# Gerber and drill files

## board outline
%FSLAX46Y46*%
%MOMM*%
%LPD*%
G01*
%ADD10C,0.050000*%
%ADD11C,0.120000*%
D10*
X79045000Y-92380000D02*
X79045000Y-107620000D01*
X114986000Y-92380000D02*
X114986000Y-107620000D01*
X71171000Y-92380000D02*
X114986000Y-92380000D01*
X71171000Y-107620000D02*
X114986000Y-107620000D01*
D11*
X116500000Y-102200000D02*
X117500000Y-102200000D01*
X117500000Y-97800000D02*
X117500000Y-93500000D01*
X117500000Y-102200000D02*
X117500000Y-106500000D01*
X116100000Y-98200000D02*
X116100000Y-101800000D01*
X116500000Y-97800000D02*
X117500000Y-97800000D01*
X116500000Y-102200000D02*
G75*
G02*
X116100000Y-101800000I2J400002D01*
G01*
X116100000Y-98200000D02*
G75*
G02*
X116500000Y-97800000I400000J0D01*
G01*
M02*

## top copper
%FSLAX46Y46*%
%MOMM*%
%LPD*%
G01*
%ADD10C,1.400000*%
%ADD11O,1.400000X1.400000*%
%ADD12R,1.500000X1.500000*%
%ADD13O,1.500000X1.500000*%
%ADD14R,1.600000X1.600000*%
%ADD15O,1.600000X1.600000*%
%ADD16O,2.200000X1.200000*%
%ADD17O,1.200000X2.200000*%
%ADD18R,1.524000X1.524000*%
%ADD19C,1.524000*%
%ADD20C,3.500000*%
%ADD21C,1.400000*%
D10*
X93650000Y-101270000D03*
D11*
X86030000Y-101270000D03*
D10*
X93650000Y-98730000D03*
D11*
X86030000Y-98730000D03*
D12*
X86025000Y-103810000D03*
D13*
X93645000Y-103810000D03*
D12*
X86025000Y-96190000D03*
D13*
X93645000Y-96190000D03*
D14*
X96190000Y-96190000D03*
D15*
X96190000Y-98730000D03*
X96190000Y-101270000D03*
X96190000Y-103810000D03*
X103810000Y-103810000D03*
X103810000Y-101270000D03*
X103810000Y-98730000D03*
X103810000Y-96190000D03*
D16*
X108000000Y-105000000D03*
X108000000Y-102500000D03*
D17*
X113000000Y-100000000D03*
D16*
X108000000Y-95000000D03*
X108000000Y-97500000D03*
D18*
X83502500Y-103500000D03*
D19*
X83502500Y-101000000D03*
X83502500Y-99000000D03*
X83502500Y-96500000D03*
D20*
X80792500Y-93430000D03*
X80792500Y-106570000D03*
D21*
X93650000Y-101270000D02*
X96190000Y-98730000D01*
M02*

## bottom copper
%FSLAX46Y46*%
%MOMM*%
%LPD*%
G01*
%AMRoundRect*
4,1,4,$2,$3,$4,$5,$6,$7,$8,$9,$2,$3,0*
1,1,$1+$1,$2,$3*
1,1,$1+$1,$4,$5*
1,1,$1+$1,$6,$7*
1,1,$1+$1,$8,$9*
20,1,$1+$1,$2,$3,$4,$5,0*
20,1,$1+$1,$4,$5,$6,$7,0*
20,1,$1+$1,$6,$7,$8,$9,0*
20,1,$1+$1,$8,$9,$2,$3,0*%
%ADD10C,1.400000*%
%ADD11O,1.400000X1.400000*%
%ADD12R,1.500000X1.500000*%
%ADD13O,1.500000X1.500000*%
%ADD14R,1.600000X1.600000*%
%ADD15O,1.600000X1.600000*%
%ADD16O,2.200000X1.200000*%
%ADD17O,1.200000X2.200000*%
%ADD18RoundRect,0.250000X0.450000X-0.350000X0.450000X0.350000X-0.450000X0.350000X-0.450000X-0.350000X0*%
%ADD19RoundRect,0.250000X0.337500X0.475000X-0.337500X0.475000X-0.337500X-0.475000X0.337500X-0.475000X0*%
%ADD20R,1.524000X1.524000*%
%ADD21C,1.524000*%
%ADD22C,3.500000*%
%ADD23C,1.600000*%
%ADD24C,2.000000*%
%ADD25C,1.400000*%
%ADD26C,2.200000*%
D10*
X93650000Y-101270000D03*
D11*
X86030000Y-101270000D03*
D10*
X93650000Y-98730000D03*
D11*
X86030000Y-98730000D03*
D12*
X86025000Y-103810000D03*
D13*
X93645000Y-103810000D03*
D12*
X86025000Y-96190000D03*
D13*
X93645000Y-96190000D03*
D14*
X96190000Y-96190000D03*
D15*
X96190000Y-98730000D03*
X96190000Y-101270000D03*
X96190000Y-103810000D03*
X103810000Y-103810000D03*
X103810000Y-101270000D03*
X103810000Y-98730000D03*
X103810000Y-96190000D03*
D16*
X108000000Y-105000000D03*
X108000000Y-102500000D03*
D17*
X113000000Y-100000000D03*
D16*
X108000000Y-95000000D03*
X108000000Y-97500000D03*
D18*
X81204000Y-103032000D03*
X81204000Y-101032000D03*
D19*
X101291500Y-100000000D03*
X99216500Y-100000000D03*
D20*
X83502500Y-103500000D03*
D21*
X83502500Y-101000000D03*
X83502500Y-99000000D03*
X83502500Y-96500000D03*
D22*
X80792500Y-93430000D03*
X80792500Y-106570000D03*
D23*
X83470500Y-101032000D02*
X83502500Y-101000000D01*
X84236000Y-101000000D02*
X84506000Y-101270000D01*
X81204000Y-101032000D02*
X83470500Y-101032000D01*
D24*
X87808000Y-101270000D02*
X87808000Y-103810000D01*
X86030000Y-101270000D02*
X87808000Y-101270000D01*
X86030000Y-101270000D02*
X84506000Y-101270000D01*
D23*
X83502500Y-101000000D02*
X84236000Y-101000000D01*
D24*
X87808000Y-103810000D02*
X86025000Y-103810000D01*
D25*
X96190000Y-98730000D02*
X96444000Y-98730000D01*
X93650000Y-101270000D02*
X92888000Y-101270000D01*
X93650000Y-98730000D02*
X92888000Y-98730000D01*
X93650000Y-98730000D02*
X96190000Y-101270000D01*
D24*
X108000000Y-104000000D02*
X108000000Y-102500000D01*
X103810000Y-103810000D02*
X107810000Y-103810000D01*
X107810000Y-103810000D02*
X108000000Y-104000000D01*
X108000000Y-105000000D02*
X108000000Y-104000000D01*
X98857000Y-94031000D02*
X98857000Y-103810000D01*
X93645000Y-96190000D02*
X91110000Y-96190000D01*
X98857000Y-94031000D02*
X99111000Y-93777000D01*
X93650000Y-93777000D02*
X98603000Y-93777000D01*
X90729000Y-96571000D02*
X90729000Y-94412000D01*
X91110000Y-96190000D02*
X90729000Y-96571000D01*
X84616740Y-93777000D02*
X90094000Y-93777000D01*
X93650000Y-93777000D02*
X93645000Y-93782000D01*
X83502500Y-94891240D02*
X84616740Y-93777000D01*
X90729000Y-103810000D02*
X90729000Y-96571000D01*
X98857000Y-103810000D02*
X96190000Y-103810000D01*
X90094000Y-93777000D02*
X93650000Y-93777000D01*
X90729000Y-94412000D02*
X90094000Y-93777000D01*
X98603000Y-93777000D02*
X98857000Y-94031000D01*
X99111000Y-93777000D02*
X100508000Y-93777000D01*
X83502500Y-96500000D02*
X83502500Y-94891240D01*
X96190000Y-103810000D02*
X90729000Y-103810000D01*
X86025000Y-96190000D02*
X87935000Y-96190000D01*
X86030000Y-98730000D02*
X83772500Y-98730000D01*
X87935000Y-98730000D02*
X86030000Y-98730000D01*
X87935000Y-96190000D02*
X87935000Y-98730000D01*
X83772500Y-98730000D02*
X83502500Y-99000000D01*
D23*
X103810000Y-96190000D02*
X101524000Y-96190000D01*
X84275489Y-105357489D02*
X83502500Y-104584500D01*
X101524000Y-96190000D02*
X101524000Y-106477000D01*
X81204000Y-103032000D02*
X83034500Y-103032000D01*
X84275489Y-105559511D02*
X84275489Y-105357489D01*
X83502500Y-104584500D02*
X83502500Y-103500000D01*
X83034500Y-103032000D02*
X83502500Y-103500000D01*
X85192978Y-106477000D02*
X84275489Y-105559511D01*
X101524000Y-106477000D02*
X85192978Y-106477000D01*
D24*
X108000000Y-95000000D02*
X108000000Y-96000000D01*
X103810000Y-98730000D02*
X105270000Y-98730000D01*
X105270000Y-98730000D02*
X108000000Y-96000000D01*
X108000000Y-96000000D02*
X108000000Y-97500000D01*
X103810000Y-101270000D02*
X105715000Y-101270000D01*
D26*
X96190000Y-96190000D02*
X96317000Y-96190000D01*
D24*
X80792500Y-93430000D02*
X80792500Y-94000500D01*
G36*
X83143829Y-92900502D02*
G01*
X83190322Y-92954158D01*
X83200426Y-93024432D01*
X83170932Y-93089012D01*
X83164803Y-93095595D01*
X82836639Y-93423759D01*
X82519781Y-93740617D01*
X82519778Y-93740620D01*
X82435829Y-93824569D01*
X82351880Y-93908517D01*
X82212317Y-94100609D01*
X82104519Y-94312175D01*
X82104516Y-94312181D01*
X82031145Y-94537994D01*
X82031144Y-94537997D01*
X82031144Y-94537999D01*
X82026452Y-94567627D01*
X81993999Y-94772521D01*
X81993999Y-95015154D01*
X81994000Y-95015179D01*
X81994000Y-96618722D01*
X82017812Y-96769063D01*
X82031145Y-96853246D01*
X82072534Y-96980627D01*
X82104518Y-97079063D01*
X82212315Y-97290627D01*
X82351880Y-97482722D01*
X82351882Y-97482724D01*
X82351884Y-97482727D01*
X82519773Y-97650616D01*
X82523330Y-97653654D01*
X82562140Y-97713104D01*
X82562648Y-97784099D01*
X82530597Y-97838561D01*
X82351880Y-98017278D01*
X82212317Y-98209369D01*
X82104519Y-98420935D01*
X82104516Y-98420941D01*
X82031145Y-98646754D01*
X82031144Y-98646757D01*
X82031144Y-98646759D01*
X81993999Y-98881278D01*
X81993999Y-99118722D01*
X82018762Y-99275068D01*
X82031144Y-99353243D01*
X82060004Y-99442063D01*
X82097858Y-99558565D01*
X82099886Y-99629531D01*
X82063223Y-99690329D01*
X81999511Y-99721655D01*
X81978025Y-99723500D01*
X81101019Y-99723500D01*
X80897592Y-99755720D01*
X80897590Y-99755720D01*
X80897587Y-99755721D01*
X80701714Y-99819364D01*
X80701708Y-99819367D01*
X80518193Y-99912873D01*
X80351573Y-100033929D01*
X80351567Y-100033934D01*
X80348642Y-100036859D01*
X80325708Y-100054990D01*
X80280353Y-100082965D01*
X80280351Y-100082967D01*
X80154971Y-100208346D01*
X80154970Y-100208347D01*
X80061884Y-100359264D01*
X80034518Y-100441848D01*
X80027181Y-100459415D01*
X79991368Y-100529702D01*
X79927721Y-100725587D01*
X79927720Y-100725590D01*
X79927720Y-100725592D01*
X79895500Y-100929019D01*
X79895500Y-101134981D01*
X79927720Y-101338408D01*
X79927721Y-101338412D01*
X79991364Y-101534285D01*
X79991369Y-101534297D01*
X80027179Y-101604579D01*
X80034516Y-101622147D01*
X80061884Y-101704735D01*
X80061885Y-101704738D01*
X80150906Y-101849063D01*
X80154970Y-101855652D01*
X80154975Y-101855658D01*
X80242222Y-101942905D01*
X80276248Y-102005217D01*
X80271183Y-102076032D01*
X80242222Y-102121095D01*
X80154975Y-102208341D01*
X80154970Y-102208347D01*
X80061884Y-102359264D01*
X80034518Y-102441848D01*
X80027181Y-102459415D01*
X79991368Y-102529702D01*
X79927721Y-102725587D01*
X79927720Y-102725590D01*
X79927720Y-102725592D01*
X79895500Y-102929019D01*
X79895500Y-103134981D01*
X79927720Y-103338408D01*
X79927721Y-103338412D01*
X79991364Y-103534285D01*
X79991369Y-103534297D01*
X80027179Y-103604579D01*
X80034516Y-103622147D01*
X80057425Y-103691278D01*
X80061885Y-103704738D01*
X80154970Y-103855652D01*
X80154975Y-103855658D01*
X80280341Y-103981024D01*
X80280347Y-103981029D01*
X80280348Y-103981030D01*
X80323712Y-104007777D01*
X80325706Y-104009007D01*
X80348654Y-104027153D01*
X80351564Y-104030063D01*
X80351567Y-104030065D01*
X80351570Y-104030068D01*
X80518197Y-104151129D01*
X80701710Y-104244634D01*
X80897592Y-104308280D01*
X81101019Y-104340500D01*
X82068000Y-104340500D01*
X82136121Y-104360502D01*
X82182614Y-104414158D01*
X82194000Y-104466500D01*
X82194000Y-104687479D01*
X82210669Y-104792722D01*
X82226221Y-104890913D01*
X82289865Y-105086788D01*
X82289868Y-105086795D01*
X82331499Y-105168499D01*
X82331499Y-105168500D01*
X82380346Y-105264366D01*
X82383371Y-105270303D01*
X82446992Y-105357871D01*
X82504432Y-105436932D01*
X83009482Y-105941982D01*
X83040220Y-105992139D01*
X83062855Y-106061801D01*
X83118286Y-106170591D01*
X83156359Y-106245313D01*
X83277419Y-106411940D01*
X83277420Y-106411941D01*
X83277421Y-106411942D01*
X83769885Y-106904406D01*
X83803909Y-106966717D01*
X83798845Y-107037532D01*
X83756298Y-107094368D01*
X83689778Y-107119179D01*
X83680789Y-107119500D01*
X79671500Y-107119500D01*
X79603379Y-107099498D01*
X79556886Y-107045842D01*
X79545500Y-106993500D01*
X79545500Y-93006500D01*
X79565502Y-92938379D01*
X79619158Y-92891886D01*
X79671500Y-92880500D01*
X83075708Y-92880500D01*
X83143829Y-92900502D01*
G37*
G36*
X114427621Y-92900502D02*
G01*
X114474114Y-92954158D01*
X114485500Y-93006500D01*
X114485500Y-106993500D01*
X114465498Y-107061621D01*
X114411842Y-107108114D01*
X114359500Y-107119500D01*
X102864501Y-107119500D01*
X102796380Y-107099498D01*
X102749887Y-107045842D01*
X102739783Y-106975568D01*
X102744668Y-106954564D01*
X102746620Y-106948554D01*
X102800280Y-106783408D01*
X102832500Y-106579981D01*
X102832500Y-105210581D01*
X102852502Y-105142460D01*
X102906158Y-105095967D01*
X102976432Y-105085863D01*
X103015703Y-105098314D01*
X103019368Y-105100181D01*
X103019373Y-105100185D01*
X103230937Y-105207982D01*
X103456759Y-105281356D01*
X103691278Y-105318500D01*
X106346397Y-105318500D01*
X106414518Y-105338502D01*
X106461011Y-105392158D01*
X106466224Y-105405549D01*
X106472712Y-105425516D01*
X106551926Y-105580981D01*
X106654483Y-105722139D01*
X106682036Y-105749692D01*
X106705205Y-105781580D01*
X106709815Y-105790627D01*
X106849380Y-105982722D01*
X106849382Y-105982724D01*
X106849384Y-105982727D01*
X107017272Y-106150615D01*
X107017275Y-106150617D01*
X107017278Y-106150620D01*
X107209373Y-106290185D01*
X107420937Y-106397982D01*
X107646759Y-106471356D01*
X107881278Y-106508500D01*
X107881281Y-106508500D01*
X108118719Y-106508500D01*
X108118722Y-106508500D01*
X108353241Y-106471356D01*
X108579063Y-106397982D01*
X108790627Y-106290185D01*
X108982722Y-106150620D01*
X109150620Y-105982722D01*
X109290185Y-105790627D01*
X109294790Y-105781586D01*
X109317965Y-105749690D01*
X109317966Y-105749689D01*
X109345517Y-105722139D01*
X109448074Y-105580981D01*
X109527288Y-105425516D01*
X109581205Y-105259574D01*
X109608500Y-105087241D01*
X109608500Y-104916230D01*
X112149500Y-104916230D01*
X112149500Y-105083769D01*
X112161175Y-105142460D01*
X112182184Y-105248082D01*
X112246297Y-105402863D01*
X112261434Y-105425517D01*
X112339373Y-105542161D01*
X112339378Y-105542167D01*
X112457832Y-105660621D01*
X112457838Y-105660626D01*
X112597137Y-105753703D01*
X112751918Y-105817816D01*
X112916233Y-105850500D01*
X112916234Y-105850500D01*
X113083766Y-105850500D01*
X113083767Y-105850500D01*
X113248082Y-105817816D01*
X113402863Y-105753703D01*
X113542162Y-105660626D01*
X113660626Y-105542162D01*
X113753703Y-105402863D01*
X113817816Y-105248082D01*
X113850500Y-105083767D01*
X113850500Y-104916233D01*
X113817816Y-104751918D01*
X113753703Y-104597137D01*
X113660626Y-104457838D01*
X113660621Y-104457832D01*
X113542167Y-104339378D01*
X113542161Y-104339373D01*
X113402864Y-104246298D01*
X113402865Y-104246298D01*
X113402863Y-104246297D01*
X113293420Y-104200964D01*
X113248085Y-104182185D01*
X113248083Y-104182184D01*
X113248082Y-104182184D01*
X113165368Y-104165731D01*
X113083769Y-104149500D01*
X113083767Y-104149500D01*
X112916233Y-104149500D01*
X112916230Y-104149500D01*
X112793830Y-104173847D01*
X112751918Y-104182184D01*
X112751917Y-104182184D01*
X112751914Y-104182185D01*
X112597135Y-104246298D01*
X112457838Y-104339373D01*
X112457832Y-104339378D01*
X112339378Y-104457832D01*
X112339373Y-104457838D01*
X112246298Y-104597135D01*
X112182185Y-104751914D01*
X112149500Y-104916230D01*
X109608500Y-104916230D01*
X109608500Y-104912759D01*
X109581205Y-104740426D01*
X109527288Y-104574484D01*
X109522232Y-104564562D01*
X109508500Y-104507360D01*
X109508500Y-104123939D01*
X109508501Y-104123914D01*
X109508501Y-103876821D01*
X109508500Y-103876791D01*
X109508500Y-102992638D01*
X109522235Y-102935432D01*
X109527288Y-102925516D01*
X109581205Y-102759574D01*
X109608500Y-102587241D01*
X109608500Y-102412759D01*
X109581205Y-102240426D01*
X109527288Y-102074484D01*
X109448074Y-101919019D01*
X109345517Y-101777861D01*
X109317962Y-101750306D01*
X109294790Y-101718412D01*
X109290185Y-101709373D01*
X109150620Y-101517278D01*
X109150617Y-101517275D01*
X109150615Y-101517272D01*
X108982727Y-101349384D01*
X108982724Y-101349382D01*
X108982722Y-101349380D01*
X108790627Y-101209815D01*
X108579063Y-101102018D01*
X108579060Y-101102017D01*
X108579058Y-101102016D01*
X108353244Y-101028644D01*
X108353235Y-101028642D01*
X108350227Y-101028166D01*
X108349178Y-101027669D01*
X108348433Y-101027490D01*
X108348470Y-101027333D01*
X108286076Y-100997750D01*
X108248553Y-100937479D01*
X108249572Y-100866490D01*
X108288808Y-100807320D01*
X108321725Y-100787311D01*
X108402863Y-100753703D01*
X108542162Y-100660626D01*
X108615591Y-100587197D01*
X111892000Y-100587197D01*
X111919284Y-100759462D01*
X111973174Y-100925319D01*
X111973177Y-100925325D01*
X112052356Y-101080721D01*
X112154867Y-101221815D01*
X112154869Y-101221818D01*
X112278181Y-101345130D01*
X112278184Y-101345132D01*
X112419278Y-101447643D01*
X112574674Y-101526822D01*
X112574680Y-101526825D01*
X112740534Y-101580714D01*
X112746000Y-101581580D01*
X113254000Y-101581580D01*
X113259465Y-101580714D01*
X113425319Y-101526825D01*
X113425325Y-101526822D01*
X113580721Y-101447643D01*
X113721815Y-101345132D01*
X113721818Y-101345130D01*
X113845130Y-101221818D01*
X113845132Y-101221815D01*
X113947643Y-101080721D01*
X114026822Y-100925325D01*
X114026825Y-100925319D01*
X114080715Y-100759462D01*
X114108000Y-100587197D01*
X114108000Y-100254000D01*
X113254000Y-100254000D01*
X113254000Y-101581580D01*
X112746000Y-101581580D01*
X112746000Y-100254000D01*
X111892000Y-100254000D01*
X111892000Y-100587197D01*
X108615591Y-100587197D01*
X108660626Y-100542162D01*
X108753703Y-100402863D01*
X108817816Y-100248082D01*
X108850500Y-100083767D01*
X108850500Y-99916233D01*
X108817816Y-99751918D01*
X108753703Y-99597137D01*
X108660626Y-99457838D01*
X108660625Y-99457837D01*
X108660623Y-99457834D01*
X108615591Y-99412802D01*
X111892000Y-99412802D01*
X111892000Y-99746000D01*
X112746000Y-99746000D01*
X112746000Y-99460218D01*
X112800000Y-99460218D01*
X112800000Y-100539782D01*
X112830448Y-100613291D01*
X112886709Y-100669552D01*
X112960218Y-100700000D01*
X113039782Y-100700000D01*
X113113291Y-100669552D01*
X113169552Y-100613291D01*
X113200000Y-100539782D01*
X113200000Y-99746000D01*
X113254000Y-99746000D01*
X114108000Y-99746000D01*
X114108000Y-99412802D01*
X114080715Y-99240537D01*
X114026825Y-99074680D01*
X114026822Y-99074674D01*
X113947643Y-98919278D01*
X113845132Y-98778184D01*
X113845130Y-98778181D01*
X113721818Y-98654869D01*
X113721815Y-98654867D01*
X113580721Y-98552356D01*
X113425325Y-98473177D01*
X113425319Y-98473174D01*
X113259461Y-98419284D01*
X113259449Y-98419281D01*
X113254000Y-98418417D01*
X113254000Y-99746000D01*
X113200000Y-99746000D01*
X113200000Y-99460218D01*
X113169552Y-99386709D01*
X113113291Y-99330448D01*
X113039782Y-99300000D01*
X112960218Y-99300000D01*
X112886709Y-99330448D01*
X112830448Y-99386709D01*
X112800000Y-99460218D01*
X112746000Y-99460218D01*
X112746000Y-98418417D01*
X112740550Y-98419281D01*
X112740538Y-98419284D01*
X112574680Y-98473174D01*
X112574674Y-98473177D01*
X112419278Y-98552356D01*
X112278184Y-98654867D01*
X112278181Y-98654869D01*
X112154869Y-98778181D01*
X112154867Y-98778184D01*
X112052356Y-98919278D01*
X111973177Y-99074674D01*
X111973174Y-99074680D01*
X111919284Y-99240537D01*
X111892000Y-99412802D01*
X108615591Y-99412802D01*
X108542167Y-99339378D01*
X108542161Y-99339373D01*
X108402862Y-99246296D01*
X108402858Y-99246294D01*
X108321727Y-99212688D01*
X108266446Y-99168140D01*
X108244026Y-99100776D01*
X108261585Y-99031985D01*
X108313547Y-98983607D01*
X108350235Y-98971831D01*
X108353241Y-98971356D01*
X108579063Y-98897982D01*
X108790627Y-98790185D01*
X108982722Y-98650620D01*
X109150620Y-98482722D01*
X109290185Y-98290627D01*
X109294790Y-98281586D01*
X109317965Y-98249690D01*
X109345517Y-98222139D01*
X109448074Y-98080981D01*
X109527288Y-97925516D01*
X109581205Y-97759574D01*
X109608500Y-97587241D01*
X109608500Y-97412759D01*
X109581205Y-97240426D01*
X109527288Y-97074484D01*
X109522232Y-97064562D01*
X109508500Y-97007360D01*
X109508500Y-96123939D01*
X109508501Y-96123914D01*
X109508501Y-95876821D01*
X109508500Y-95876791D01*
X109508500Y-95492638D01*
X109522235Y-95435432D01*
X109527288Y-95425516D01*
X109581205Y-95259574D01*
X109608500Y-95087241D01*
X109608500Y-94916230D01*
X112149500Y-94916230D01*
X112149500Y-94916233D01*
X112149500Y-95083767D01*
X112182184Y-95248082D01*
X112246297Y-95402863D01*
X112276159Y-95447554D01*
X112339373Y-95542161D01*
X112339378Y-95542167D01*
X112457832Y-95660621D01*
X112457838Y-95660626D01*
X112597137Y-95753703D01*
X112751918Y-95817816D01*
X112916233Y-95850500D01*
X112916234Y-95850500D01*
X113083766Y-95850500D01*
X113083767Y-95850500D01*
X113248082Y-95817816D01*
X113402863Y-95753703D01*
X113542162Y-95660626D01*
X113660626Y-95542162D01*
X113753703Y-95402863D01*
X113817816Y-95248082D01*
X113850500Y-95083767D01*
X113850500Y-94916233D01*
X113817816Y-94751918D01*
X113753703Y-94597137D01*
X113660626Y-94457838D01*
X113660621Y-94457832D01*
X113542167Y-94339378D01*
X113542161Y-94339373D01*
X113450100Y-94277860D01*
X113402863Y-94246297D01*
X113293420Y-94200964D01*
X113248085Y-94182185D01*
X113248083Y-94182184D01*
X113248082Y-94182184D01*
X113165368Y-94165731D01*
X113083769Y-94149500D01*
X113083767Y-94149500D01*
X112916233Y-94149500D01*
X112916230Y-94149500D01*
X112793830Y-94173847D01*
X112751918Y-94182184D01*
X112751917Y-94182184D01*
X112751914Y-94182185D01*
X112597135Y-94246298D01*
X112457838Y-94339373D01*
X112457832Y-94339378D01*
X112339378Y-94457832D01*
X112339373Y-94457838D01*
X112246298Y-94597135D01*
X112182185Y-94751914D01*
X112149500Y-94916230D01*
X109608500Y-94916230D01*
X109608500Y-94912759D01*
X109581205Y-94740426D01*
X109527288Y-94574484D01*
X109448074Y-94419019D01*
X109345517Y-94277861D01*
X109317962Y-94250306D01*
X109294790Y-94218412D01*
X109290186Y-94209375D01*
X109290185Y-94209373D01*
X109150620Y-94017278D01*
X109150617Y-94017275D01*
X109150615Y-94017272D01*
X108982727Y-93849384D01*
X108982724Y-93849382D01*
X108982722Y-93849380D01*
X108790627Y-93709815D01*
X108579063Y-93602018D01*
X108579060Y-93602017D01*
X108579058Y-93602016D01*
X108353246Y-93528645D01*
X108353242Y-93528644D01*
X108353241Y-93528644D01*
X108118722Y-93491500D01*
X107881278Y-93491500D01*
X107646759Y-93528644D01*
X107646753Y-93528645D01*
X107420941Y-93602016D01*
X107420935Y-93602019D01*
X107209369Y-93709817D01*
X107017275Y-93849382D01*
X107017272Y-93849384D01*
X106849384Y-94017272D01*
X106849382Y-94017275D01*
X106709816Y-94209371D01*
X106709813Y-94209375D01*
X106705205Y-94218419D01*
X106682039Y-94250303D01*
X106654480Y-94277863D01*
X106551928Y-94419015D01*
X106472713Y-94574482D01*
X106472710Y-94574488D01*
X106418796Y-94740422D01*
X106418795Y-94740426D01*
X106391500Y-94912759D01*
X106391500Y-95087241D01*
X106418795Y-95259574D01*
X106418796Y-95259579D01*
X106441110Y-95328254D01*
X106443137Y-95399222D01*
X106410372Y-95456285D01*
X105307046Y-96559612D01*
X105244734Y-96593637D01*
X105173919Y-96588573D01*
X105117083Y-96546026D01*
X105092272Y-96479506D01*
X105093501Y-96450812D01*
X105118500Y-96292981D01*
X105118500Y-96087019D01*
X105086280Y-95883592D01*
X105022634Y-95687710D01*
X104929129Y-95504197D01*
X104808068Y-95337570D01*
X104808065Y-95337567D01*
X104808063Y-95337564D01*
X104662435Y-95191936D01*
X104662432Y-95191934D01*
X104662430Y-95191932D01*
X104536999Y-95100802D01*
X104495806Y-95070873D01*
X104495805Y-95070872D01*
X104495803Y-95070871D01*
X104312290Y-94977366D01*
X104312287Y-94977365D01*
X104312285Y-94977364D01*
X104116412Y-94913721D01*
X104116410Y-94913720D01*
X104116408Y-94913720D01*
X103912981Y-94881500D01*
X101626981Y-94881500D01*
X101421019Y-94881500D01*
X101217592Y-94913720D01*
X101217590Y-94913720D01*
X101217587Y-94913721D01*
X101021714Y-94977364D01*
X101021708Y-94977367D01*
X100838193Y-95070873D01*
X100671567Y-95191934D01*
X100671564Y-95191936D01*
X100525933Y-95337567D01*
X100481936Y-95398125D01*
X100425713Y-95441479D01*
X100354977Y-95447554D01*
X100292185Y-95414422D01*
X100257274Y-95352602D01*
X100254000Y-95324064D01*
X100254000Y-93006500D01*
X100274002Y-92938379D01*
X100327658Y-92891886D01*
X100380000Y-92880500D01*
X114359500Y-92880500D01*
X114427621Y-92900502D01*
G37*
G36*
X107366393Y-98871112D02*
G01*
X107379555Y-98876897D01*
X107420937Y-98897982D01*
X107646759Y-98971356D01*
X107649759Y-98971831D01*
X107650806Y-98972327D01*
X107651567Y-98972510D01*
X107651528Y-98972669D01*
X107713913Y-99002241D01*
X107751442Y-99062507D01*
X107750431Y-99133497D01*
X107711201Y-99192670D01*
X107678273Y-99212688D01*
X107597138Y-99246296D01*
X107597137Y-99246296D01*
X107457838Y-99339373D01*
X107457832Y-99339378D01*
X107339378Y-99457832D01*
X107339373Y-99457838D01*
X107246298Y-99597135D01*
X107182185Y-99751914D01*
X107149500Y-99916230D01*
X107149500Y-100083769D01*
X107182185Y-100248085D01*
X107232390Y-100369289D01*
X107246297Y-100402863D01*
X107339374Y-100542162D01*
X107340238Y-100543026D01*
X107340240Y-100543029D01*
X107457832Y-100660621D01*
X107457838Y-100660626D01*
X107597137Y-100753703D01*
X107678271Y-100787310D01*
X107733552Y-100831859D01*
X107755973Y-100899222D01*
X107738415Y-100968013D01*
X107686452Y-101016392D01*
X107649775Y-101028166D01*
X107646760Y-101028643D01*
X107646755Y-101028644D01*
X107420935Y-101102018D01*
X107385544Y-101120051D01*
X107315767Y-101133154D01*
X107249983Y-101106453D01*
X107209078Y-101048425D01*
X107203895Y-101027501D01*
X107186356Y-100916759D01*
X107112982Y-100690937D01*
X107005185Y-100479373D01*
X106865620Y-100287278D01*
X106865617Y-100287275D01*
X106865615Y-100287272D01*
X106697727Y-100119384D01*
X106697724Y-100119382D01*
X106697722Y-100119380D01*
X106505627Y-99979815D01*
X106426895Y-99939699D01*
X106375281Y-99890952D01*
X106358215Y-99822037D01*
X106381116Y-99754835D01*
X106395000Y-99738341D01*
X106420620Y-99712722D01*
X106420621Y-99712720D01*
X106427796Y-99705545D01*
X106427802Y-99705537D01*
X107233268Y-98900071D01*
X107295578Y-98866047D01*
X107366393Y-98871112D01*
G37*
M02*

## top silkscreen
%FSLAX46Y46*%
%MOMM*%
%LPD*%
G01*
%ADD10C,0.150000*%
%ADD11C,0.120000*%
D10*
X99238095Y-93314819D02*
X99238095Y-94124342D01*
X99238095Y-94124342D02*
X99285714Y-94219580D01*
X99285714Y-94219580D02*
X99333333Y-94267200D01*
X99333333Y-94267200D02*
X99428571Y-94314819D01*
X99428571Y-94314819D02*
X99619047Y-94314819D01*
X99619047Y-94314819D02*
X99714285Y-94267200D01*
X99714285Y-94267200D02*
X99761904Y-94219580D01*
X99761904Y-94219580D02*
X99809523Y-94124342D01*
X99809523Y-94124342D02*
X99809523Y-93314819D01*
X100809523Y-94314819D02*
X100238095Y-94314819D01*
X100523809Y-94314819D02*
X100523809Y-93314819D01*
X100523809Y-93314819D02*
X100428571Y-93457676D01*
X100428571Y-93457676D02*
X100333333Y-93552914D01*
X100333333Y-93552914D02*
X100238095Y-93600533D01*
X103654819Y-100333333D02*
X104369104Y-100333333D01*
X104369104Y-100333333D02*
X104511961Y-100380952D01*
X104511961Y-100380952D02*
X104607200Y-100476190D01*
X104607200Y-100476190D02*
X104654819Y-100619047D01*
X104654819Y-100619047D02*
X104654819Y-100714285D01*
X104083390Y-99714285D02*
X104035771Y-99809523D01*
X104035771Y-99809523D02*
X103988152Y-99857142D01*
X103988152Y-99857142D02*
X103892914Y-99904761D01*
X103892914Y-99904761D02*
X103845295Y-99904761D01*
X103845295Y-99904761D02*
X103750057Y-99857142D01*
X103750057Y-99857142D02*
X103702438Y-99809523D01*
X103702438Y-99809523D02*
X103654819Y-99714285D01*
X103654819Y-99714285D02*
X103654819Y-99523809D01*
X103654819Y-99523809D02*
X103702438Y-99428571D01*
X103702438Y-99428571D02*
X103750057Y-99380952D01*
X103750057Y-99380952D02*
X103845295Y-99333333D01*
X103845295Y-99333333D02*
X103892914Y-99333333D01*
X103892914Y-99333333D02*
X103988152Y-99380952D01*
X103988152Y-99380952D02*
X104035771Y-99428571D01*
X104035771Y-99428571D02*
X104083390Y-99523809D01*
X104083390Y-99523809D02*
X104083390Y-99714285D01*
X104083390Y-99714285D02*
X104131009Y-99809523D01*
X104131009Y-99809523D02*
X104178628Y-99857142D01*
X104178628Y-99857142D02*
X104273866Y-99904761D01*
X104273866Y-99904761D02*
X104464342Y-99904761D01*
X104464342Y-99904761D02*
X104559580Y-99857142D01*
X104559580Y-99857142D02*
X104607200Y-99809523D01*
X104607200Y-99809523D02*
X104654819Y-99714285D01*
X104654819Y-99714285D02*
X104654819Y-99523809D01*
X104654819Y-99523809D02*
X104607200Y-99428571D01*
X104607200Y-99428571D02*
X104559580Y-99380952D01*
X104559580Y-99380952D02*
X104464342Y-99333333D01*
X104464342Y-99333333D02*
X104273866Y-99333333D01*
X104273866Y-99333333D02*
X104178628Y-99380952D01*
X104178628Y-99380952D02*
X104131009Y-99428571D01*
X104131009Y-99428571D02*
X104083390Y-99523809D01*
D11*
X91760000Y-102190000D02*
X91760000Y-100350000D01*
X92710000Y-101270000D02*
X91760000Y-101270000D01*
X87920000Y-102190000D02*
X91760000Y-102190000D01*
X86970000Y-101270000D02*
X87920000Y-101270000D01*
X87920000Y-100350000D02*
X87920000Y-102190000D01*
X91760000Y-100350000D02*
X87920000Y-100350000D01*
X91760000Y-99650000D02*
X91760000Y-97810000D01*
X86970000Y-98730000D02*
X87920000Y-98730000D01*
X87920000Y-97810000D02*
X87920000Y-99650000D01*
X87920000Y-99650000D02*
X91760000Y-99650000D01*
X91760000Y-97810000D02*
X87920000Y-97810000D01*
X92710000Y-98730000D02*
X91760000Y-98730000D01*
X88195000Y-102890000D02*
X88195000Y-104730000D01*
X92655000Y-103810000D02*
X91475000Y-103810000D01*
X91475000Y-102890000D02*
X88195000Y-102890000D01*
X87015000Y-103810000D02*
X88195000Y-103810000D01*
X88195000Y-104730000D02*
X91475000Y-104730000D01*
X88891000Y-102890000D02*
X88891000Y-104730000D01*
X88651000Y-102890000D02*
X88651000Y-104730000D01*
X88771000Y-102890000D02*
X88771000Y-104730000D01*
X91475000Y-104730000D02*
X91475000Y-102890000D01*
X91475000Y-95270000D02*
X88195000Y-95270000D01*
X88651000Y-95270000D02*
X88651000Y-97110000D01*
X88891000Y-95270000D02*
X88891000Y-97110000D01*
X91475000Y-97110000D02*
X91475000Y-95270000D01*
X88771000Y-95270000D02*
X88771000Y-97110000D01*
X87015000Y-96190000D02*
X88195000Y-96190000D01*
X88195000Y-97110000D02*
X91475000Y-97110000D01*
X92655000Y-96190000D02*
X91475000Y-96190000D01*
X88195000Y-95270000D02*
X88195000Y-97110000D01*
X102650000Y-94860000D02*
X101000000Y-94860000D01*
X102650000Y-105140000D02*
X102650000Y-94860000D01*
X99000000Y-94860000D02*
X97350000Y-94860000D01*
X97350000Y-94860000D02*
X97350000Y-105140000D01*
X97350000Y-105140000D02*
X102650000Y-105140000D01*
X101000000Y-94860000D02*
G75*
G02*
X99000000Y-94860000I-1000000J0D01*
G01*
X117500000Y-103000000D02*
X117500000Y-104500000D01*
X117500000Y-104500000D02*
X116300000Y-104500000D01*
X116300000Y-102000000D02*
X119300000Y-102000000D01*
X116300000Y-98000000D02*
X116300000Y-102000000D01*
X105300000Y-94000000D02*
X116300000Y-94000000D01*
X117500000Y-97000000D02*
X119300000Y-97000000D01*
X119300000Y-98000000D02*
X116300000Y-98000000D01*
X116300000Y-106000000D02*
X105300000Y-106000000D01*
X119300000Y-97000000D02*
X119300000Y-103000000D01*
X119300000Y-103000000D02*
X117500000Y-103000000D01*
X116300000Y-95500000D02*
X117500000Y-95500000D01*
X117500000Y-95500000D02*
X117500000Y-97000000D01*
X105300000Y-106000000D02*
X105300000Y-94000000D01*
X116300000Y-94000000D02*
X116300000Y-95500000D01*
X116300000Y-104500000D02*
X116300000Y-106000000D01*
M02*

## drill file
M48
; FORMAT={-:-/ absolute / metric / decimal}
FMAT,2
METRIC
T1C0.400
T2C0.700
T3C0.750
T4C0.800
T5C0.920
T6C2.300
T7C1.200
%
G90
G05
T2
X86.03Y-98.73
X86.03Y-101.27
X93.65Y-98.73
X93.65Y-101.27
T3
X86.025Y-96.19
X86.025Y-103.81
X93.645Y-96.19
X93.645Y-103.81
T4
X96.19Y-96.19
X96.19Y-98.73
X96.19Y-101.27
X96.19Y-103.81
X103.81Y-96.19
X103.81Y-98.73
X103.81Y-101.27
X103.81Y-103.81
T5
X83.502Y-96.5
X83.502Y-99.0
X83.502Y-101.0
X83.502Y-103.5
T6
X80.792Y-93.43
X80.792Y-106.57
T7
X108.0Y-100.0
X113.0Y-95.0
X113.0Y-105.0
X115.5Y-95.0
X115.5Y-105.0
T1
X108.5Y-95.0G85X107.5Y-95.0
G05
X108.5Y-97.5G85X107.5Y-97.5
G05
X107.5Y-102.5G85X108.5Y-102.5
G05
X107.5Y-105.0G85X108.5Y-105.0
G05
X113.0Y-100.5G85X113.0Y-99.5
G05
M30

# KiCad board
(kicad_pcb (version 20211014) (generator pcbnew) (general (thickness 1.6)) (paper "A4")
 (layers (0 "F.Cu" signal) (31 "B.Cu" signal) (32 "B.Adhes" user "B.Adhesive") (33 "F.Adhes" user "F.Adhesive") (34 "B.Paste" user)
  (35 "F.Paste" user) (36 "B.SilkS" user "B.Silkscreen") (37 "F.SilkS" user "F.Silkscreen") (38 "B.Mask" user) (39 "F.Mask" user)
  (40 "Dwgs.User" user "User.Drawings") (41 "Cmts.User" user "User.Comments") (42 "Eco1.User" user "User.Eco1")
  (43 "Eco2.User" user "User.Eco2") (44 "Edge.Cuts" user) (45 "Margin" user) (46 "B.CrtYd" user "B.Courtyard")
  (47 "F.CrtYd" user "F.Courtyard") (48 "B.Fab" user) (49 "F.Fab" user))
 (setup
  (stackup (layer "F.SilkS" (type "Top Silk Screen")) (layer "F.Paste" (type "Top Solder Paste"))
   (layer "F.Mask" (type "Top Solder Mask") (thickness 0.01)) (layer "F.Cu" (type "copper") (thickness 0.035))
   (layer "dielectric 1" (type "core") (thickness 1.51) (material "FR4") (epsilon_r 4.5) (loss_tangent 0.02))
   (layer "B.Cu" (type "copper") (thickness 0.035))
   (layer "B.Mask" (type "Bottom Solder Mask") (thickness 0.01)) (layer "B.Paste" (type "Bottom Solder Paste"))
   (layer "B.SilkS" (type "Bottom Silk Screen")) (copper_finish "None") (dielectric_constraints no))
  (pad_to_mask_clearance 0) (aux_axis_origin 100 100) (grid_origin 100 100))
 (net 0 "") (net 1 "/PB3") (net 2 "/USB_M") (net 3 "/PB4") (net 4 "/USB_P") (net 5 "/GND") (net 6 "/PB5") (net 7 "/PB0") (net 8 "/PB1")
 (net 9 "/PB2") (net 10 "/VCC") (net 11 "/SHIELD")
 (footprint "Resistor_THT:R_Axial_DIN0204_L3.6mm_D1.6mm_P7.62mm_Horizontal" (layer "F.Cu") (at 93.65 101.27 180)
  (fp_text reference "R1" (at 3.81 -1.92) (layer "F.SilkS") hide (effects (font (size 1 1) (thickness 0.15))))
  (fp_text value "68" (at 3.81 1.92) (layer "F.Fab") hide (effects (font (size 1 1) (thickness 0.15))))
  (fp_line (start 1.89 -0.92) (end 1.89 0.92) (layer "F.SilkS") (width 0.12))
  (fp_line (start 0.94 0) (end 1.89 0) (layer "F.SilkS") (width 0.12))
  (fp_line (start 5.73 -0.92) (end 1.89 -0.92) (layer "F.SilkS") (width 0.12))
  (fp_line (start 6.68 0) (end 5.73 0) (layer "F.SilkS") (width 0.12))
  (fp_line (start 5.73 0.92) (end 5.73 -0.92) (layer "F.SilkS") (width 0.12))
  (fp_line (start 1.89 0.92) (end 5.73 0.92) (layer "F.SilkS") (width 0.12))
  (pad "1" thru_hole circle locked (at 0 0 180) (size 1.4 1.4) (drill 0.7) (layers *.Cu *.Mask) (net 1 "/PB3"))
  (pad "2" thru_hole oval locked (at 7.62 0 180) (size 1.4 1.4) (drill 0.7) (layers *.Cu *.Mask) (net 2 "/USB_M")))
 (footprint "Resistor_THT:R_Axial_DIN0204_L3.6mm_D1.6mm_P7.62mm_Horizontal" (layer "F.Cu") (at 93.65 98.73 180)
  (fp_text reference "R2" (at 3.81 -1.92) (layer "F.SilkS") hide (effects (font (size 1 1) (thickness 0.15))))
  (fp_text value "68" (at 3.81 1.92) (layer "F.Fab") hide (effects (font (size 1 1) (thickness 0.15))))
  (fp_line (start 1.89 -0.92) (end 1.89 0.92) (layer "F.SilkS") (width 0.12))
  (fp_line (start 6.68 0) (end 5.73 0) (layer "F.SilkS") (width 0.12))
  (fp_line (start 5.73 0.92) (end 5.73 -0.92) (layer "F.SilkS") (width 0.12))
  (fp_line (start 5.73 -0.92) (end 1.89 -0.92) (layer "F.SilkS") (width 0.12))
  (fp_line (start 1.89 0.92) (end 5.73 0.92) (layer "F.SilkS") (width 0.12))
  (fp_line (start 0.94 0) (end 1.89 0) (layer "F.SilkS") (width 0.12))
  (pad "1" thru_hole circle locked (at 0 0 180) (size 1.4 1.4) (drill 0.7) (layers *.Cu *.Mask) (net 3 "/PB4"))
  (pad "2" thru_hole oval locked (at 7.62 0 180) (size 1.4 1.4) (drill 0.7) (layers *.Cu *.Mask) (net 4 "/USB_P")))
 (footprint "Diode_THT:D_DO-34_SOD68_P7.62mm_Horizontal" (layer "F.Cu") (at 86.025 103.81)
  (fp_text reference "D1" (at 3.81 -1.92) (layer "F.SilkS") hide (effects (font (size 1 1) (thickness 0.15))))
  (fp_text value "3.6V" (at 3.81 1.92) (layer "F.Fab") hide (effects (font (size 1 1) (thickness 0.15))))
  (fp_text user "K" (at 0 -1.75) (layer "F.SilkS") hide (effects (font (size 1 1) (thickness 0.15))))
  (fp_line (start 2.17 -0.92) (end 2.17 0.92) (layer "F.SilkS") (width 0.12))
  (fp_line (start 6.63 0) (end 5.45 0) (layer "F.SilkS") (width 0.12))
  (fp_line (start 5.45 -0.92) (end 2.17 -0.92) (layer "F.SilkS") (width 0.12))
  (fp_line (start 0.99 0) (end 2.17 0) (layer "F.SilkS") (width 0.12))
  (fp_line (start 2.17 0.92) (end 5.45 0.92) (layer "F.SilkS") (width 0.12))
  (fp_line (start 2.866 -0.92) (end 2.866 0.92) (layer "F.SilkS") (width 0.12))
  (fp_line (start 2.626 -0.92) (end 2.626 0.92) (layer "F.SilkS") (width 0.12))
  (fp_line (start 2.746 -0.92) (end 2.746 0.92) (layer "F.SilkS") (width 0.12))
  (fp_line (start 5.45 0.92) (end 5.45 -0.92) (layer "F.SilkS") (width 0.12))
  (pad "1" thru_hole rect locked (at 0 0) (size 1.5 1.5) (drill 0.75) (layers *.Cu *.Mask) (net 2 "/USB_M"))
  (pad "2" thru_hole oval locked (at 7.62 0) (size 1.5 1.5) (drill 0.75) (layers *.Cu *.Mask) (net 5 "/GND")))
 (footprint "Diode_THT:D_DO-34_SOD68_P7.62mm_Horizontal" (layer "F.Cu") (at 86.025 96.19)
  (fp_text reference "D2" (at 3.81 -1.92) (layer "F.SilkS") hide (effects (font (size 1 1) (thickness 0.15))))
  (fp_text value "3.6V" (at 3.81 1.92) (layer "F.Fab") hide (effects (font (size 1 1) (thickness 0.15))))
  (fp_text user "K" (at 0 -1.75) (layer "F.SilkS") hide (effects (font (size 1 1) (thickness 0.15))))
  (fp_line (start 5.45 -0.92) (end 2.17 -0.92) (layer "F.SilkS") (width 0.12))
  (fp_line (start 2.626 -0.92) (end 2.626 0.92) (layer "F.SilkS") (width 0.12))
  (fp_line (start 2.866 -0.92) (end 2.866 0.92) (layer "F.SilkS") (width 0.12))
  (fp_line (start 5.45 0.92) (end 5.45 -0.92) (layer "F.SilkS") (width 0.12))
  (fp_line (start 2.746 -0.92) (end 2.746 0.92) (layer "F.SilkS") (width 0.12))
  (fp_line (start 0.99 0) (end 2.17 0) (layer "F.SilkS") (width 0.12))
  (fp_line (start 2.17 0.92) (end 5.45 0.92) (layer "F.SilkS") (width 0.12))
  (fp_line (start 6.63 0) (end 5.45 0) (layer "F.SilkS") (width 0.12))
  (fp_line (start 2.17 -0.92) (end 2.17 0.92) (layer "F.SilkS") (width 0.12))
  (pad "1" thru_hole rect locked (at 0 0) (size 1.5 1.5) (drill 0.75) (layers *.Cu *.Mask) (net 4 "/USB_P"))
  (pad "2" thru_hole oval locked (at 7.62 0) (size 1.5 1.5) (drill 0.75) (layers *.Cu *.Mask) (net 5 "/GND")))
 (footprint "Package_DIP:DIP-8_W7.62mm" (layer "F.Cu") (at 96.19 96.19)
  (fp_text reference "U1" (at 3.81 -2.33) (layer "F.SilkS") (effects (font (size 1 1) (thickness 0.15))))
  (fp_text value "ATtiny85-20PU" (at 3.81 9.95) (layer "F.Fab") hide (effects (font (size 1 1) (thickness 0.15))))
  (fp_line (start 6.46 -1.33) (end 4.81 -1.33) (layer "F.SilkS") (width 0.12))
  (fp_line (start 6.46 8.95) (end 6.46 -1.33) (layer "F.SilkS") (width 0.12))
  (fp_line (start 2.81 -1.33) (end 1.16 -1.33) (layer "F.SilkS") (width 0.12))
  (fp_line (start 1.16 -1.33) (end 1.16 8.95) (layer "F.SilkS") (width 0.12))
  (fp_line (start 1.16 8.95) (end 6.46 8.95) (layer "F.SilkS") (width 0.12))
  (fp_arc (start 4.81 -1.33) (mid 3.81 -0.33) (end 2.81 -1.33) (layer "F.SilkS") (width 0.12))
  (pad "1" thru_hole rect locked (at 0 0) (size 1.6 1.6) (drill 0.8) (layers *.Cu *.Mask) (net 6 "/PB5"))
  (pad "2" thru_hole oval locked (at 0 2.54) (size 1.6 1.6) (drill 0.8) (layers *.Cu *.Mask) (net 1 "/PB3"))
  (pad "3" thru_hole oval locked (at 0 5.08) (size 1.6 1.6) (drill 0.8) (layers *.Cu *.Mask) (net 3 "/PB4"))
  (pad "4" thru_hole oval locked (at 0 7.62) (size 1.6 1.6) (drill 0.8) (layers *.Cu *.Mask) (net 5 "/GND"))
  (pad "5" thru_hole oval locked (at 7.62 7.62) (size 1.6 1.6) (drill 0.8) (layers *.Cu *.Mask) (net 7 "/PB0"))
  (pad "6" thru_hole oval locked (at 7.62 5.08) (size 1.6 1.6) (drill 0.8) (layers *.Cu *.Mask) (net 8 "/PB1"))
  (pad "7" thru_hole oval locked (at 7.62 2.54) (size 1.6 1.6) (drill 0.8) (layers *.Cu *.Mask) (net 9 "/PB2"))
  (pad "8" thru_hole oval locked (at 7.62 0) (size 1.6 1.6) (drill 0.8) (layers *.Cu *.Mask) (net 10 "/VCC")))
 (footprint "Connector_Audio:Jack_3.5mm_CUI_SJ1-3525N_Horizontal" (layer "F.Cu") (at 113 100 90)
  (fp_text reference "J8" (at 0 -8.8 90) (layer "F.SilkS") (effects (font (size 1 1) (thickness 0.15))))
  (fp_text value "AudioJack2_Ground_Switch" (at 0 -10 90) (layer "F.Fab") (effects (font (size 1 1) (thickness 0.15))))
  (fp_line (start -3 4.5) (end -4.5 4.5) (layer "F.SilkS") (width 0.12))
  (fp_line (start -4.5 4.5) (end -4.5 3.3) (layer "F.SilkS") (width 0.12))
  (fp_line (start -2 3.3) (end -2 6.3) (layer "F.SilkS") (width 0.12))
  (fp_line (start 2 3.3) (end -2 3.3) (layer "F.SilkS") (width 0.12))
  (fp_line (start 6 -7.7) (end 6 3.3) (layer "F.SilkS") (width 0.12))
  (fp_line (start 3 4.5) (end 3 6.3) (layer "F.SilkS") (width 0.12))
  (fp_line (start 2 6.3) (end 2 3.3) (layer "F.SilkS") (width 0.12))
  (fp_line (start -6 3.3) (end -6 -7.7) (layer "F.SilkS") (width 0.12))
  (fp_line (start 3 6.3) (end -3 6.3) (layer "F.SilkS") (width 0.12))
  (fp_line (start -3 6.3) (end -3 4.5) (layer "F.SilkS") (width 0.12))
  (fp_line (start 4.5 3.3) (end 4.5 4.5) (layer "F.SilkS") (width 0.12))
  (fp_line (start 4.5 4.5) (end 3 4.5) (layer "F.SilkS") (width 0.12))
  (fp_line (start -6 -7.7) (end 6 -7.7) (layer "F.SilkS") (width 0.12))
  (fp_line (start 6 3.3) (end 4.5 3.3) (layer "F.SilkS") (width 0.12))
  (fp_line (start -4.5 3.3) (end -6 3.3) (layer "F.SilkS") (width 0.12))
  (fp_line (start -2.2 3.5) (end -2.2 4.5) (layer "Edge.Cuts") (width 0.12))
  (fp_line (start 2.2 4.5) (end 6.5 4.5) (layer "Edge.Cuts") (width 0.12))
  (fp_line (start -2.2 4.5) (end -6.5 4.5) (layer "Edge.Cuts") (width 0.12))
  (fp_line (start 1.8 3.1) (end -1.8 3.1) (layer "Edge.Cuts") (width 0.12))
  (fp_line (start 2.2 3.5) (end 2.2 4.5) (layer "Edge.Cuts") (width 0.12))
  (fp_arc (start -2.2 3.5) (mid -2.082842 3.217158) (end -1.8 3.1) (layer "Edge.Cuts") (width 0.12))
  (fp_arc (start 1.8 3.1) (mid 2.082843 3.217157) (end 2.2 3.5) (layer "Edge.Cuts") (width 0.12))
  (pad "" np_thru_hole circle (at 5 2.5 90) (size 1.2 1.2) (drill 1.2) (layers *.Cu))
  (pad "" np_thru_hole circle (at 5 0 90) (size 1.2 1.2) (drill 1.2) (layers *.Cu))
  (pad "" np_thru_hole circle (at -5 2.5 90) (size 1.2 1.2) (drill 1.2) (layers *.Cu))
  (pad "" np_thru_hole circle (at -5 0 90) (size 1.2 1.2) (drill 1.2) (layers *.Cu))
  (pad "" np_thru_hole circle (at 0 -5 90) (size 1.2 1.2) (drill 1.2) (layers *.Cu))
  (pad "R" thru_hole oval (at -5 -5 90) (size 1.2 2.2) (drill oval 0.4 1.4) (layers *.Cu *.Mask) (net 7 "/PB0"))
  (pad "RN" thru_hole oval (at -2.5 -5 90) (size 1.2 2.2) (drill oval 0.4 1.4) (layers *.Cu *.Mask) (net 7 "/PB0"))
  (pad "S" thru_hole oval (at 0 0 90) (size 2.2 1.2) (drill oval 1.4 0.4) (layers *.Cu *.Mask) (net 5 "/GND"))
  (pad "T" thru_hole oval (at 5 -5 270) (size 1.2 2.2) (drill oval 0.4 1.4) (layers *.Cu *.Mask) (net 9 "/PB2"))
  (pad "TN" thru_hole oval (at 2.5 -5 270) (size 1.2 2.2) (drill oval 0.4 1.4) (layers *.Cu *.Mask) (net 9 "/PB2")))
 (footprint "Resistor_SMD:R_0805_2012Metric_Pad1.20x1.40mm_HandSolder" (layer "B.Cu") (at 81.204 102.032 90)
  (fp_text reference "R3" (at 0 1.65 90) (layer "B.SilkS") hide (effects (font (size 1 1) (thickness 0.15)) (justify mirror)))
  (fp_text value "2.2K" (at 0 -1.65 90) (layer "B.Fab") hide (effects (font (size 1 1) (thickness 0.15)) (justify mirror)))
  (pad "1" smd roundrect locked (at -1 0 90) (size 1.2 1.4) (layers "B.Cu" "B.Paste" "B.Mask") (roundrect_rratio 0.2083333333)
   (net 10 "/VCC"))
  (pad "2" smd roundrect locked (at 1 0 90) (size 1.2 1.4) (layers "B.Cu" "B.Paste" "B.Mask") (roundrect_rratio 0.2083333333)
   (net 2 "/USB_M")))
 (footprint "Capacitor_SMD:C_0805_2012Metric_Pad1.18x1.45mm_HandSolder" (layer "B.Cu") (at 100.254 100 180)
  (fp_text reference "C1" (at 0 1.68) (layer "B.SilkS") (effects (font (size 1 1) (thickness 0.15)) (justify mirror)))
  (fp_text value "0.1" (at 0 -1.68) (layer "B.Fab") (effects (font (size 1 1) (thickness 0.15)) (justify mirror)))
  (pad "1" smd roundrect locked (at -1.0375 0 180) (size 1.175 1.45) (layers "B.Cu" "B.Paste" "B.Mask") (roundrect_rratio 0.2127659574)
   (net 10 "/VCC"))
  (pad "2" smd roundrect locked (at 1.0375 0 180) (size 1.175 1.45) (layers "B.Cu" "B.Paste" "B.Mask") (roundrect_rratio 0.2127659574)
   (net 5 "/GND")))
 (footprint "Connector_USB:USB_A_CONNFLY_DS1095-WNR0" (layer "B.Cu") (at 83.5025 103.5 90)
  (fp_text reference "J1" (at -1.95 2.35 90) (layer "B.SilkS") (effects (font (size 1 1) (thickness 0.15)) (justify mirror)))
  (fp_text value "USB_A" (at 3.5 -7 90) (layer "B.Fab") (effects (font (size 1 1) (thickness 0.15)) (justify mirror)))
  (pad "1" thru_hole rect (at 0 0 90) (size 1.524 1.524) (drill 0.92) (layers *.Cu *.Mask) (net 10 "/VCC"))
  (pad "2" thru_hole circle (at 2.5 0 90) (size 1.524 1.524) (drill 0.92) (layers *.Cu *.Mask) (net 2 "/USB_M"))
  (pad "3" thru_hole circle (at 4.5 0 90) (size 1.524 1.524) (drill 0.92) (layers *.Cu *.Mask) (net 4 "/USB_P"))
  (pad "4" thru_hole circle (at 7 0 90) (size 1.524 1.524) (drill 0.92) (layers *.Cu *.Mask) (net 5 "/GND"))
  (pad "5" thru_hole circle (at 10.07 -2.71 90) (size 3.5 3.5) (drill 2.3) (layers *.Cu *.Mask) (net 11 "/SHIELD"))
  (pad "5" thru_hole circle (at -3.07 -2.71 90) (size 3.5 3.5) (drill 2.3) (layers *.Cu *.Mask) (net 11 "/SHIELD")))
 (gr_line (start 79.045 92.38) (end 79.045 107.62) (layer "Edge.Cuts") (width 0.05))
 (gr_line (start 114.986 92.38) (end 114.986 107.62) (layer "Edge.Cuts") (width 0.05))
 (gr_line (start 71.171 92.38) (end 114.986 92.38) (layer "Edge.Cuts") (width 0.05))
 (gr_line (start 71.171 107.62) (end 114.986 107.62) (layer "Edge.Cuts") (width 0.05))
 (segment (start 83.4705 101.032) (end 83.5025 101) (width 1.6) (layer "B.Cu") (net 2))
 (segment (start 84.236 101) (end 84.506 101.27) (width 1.6) (layer "B.Cu") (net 2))
 (segment (start 81.204 101.032) (end 83.4705 101.032) (width 1.6) (layer "B.Cu") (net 2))
 (segment (start 87.808 101.27) (end 87.808 103.81) (width 2) (layer "B.Cu") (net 2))
 (segment (start 86.03 101.27) (end 87.808 101.27) (width 2) (layer "B.Cu") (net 2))
 (segment (start 86.03 101.27) (end 84.506 101.27) (width 2) (layer "B.Cu") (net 2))
 (segment (start 83.5025 101) (end 84.236 101) (width 1.6) (layer "B.Cu") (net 2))
 (segment (start 87.808 103.81) (end 86.025 103.81) (width 2) (layer "B.Cu") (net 2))
 (segment (start 93.65 101.27) (end 96.19 98.73) (width 1.4) (layer "F.Cu") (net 1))
 (segment (start 96.19 98.73) (end 96.444 98.73) (width 1.4) (layer "B.Cu") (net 1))
 (segment (start 93.65 101.27) (end 92.888 101.27) (width 1.4) (layer "B.Cu") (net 1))
 (segment (start 93.65 98.73) (end 92.888 98.73) (width 1.4) (layer "B.Cu") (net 3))
 (segment (start 93.65 98.73) (end 96.19 101.27) (width 1.4) (layer "B.Cu") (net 3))
 (segment (start 108 104) (end 108 102.5) (width 2) (layer "B.Cu") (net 7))
 (segment (start 103.81 103.81) (end 107.81 103.81) (width 2) (layer "B.Cu") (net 7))
 (segment (start 107.81 103.81) (end 108 104) (width 2) (layer "B.Cu") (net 7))
 (segment (start 108 105) (end 108 104) (width 2) (layer "B.Cu") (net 7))
 (segment (start 98.857 94.031) (end 98.857 103.81) (width 2) (layer "B.Cu") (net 5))
 (segment (start 93.645 96.19) (end 91.11 96.19) (width 2) (layer "B.Cu") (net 5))
 (segment (start 98.857 94.031) (end 99.111 93.777) (width 2) (layer "B.Cu") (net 5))
 (segment (start 93.65 93.777) (end 98.603 93.777) (width 2) (layer "B.Cu") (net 5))
 (segment (start 90.729 96.571) (end 90.729 94.412) (width 2) (layer "B.Cu") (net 5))
 (segment (start 91.11 96.19) (end 90.729 96.571) (width 2) (layer "B.Cu") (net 5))
 (segment (start 84.61674 93.777) (end 90.094 93.777) (width 2) (layer "B.Cu") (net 5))
 (segment (start 93.65 93.777) (end 93.645 93.782) (width 2) (layer "B.Cu") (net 5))
 (segment (start 83.5025 94.89124) (end 84.61674 93.777) (width 2) (layer "B.Cu") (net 5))
 (segment (start 90.729 103.81) (end 90.729 96.571) (width 2) (layer "B.Cu") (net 5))
 (segment (start 98.857 103.81) (end 96.19 103.81) (width 2) (layer "B.Cu") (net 5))
 (segment (start 90.094 93.777) (end 93.65 93.777) (width 2) (layer "B.Cu") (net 5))
 (segment (start 90.729 94.412) (end 90.094 93.777) (width 2) (layer "B.Cu") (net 5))
 (segment (start 98.603 93.777) (end 98.857 94.031) (width 2) (layer "B.Cu") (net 5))
 (segment (start 99.111 93.777) (end 100.508 93.777) (width 2) (layer "B.Cu") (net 5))
 (segment (start 83.5025 96.5) (end 83.5025 94.89124) (width 2) (layer "B.Cu") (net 5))
 (segment (start 96.19 103.81) (end 90.729 103.81) (width 2) (layer "B.Cu") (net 5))
 (segment (start 86.025 96.19) (end 87.935 96.19) (width 2) (layer "B.Cu") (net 4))
 (segment (start 86.03 98.73) (end 83.7725 98.73) (width 2) (layer "B.Cu") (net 4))
 (segment (start 87.935 98.73) (end 86.03 98.73) (width 2) (layer "B.Cu") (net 4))
 (segment (start 87.935 96.19) (end 87.935 98.73) (width 2) (layer "B.Cu") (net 4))
 (segment (start 83.7725 98.73) (end 83.5025 99) (width 2) (layer "B.Cu") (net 4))
 (segment (start 103.81 96.19) (end 101.524 96.19) (width 1.6) (layer "B.Cu") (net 10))
 (segment (start 84.275489 105.357489) (end 83.5025 104.5845) (width 1.6) (layer "B.Cu") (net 10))
 (segment (start 101.524 96.19) (end 101.524 106.477) (width 1.6) (layer "B.Cu") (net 10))
 (segment (start 81.204 103.032) (end 83.0345 103.032) (width 1.6) (layer "B.Cu") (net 10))
 (segment (start 84.275489 105.559511) (end 84.275489 105.357489) (width 1.6) (layer "B.Cu") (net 10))
 (segment (start 83.5025 104.5845) (end 83.5025 103.5) (width 1.6) (layer "B.Cu") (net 10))
 (segment (start 83.0345 103.032) (end 83.5025 103.5) (width 1.6) (layer "B.Cu") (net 10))
 (segment (start 85.192978 106.477) (end 84.275489 105.559511) (width 1.6) (layer "B.Cu") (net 10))
 (segment (start 101.524 106.477) (end 85.192978 106.477) (width 1.6) (layer "B.Cu") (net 10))
 (segment (start 108 95) (end 108 96) (width 2) (layer "B.Cu") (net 9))
 (segment (start 103.81 98.73) (end 105.27 98.73) (width 2) (layer "B.Cu") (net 9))
 (segment (start 105.27 98.73) (end 108 96) (width 2) (layer "B.Cu") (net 9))
 (segment (start 108 96) (end 108 97.5) (width 2) (layer "B.Cu") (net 9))
 (segment (start 103.81 101.27) (end 105.715 101.27) (width 2) (layer "B.Cu") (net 8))
 (segment (start 96.19 96.19) (end 96.317 96.19) (width 2.2) (layer "B.Cu") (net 6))
 (segment (start 80.7925 93.43) (end 80.7925 94.0005) (width 2) (layer "B.Cu") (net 11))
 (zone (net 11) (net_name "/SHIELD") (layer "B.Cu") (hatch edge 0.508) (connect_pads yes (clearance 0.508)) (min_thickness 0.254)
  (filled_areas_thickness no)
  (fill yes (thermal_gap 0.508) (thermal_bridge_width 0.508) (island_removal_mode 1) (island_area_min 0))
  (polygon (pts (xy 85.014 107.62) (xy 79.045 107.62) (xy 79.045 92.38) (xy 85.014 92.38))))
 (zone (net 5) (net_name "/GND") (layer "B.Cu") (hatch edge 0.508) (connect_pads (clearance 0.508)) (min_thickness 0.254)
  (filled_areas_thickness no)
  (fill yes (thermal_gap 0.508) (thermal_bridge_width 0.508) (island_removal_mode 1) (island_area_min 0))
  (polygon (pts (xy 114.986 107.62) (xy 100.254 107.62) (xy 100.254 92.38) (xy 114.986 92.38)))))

